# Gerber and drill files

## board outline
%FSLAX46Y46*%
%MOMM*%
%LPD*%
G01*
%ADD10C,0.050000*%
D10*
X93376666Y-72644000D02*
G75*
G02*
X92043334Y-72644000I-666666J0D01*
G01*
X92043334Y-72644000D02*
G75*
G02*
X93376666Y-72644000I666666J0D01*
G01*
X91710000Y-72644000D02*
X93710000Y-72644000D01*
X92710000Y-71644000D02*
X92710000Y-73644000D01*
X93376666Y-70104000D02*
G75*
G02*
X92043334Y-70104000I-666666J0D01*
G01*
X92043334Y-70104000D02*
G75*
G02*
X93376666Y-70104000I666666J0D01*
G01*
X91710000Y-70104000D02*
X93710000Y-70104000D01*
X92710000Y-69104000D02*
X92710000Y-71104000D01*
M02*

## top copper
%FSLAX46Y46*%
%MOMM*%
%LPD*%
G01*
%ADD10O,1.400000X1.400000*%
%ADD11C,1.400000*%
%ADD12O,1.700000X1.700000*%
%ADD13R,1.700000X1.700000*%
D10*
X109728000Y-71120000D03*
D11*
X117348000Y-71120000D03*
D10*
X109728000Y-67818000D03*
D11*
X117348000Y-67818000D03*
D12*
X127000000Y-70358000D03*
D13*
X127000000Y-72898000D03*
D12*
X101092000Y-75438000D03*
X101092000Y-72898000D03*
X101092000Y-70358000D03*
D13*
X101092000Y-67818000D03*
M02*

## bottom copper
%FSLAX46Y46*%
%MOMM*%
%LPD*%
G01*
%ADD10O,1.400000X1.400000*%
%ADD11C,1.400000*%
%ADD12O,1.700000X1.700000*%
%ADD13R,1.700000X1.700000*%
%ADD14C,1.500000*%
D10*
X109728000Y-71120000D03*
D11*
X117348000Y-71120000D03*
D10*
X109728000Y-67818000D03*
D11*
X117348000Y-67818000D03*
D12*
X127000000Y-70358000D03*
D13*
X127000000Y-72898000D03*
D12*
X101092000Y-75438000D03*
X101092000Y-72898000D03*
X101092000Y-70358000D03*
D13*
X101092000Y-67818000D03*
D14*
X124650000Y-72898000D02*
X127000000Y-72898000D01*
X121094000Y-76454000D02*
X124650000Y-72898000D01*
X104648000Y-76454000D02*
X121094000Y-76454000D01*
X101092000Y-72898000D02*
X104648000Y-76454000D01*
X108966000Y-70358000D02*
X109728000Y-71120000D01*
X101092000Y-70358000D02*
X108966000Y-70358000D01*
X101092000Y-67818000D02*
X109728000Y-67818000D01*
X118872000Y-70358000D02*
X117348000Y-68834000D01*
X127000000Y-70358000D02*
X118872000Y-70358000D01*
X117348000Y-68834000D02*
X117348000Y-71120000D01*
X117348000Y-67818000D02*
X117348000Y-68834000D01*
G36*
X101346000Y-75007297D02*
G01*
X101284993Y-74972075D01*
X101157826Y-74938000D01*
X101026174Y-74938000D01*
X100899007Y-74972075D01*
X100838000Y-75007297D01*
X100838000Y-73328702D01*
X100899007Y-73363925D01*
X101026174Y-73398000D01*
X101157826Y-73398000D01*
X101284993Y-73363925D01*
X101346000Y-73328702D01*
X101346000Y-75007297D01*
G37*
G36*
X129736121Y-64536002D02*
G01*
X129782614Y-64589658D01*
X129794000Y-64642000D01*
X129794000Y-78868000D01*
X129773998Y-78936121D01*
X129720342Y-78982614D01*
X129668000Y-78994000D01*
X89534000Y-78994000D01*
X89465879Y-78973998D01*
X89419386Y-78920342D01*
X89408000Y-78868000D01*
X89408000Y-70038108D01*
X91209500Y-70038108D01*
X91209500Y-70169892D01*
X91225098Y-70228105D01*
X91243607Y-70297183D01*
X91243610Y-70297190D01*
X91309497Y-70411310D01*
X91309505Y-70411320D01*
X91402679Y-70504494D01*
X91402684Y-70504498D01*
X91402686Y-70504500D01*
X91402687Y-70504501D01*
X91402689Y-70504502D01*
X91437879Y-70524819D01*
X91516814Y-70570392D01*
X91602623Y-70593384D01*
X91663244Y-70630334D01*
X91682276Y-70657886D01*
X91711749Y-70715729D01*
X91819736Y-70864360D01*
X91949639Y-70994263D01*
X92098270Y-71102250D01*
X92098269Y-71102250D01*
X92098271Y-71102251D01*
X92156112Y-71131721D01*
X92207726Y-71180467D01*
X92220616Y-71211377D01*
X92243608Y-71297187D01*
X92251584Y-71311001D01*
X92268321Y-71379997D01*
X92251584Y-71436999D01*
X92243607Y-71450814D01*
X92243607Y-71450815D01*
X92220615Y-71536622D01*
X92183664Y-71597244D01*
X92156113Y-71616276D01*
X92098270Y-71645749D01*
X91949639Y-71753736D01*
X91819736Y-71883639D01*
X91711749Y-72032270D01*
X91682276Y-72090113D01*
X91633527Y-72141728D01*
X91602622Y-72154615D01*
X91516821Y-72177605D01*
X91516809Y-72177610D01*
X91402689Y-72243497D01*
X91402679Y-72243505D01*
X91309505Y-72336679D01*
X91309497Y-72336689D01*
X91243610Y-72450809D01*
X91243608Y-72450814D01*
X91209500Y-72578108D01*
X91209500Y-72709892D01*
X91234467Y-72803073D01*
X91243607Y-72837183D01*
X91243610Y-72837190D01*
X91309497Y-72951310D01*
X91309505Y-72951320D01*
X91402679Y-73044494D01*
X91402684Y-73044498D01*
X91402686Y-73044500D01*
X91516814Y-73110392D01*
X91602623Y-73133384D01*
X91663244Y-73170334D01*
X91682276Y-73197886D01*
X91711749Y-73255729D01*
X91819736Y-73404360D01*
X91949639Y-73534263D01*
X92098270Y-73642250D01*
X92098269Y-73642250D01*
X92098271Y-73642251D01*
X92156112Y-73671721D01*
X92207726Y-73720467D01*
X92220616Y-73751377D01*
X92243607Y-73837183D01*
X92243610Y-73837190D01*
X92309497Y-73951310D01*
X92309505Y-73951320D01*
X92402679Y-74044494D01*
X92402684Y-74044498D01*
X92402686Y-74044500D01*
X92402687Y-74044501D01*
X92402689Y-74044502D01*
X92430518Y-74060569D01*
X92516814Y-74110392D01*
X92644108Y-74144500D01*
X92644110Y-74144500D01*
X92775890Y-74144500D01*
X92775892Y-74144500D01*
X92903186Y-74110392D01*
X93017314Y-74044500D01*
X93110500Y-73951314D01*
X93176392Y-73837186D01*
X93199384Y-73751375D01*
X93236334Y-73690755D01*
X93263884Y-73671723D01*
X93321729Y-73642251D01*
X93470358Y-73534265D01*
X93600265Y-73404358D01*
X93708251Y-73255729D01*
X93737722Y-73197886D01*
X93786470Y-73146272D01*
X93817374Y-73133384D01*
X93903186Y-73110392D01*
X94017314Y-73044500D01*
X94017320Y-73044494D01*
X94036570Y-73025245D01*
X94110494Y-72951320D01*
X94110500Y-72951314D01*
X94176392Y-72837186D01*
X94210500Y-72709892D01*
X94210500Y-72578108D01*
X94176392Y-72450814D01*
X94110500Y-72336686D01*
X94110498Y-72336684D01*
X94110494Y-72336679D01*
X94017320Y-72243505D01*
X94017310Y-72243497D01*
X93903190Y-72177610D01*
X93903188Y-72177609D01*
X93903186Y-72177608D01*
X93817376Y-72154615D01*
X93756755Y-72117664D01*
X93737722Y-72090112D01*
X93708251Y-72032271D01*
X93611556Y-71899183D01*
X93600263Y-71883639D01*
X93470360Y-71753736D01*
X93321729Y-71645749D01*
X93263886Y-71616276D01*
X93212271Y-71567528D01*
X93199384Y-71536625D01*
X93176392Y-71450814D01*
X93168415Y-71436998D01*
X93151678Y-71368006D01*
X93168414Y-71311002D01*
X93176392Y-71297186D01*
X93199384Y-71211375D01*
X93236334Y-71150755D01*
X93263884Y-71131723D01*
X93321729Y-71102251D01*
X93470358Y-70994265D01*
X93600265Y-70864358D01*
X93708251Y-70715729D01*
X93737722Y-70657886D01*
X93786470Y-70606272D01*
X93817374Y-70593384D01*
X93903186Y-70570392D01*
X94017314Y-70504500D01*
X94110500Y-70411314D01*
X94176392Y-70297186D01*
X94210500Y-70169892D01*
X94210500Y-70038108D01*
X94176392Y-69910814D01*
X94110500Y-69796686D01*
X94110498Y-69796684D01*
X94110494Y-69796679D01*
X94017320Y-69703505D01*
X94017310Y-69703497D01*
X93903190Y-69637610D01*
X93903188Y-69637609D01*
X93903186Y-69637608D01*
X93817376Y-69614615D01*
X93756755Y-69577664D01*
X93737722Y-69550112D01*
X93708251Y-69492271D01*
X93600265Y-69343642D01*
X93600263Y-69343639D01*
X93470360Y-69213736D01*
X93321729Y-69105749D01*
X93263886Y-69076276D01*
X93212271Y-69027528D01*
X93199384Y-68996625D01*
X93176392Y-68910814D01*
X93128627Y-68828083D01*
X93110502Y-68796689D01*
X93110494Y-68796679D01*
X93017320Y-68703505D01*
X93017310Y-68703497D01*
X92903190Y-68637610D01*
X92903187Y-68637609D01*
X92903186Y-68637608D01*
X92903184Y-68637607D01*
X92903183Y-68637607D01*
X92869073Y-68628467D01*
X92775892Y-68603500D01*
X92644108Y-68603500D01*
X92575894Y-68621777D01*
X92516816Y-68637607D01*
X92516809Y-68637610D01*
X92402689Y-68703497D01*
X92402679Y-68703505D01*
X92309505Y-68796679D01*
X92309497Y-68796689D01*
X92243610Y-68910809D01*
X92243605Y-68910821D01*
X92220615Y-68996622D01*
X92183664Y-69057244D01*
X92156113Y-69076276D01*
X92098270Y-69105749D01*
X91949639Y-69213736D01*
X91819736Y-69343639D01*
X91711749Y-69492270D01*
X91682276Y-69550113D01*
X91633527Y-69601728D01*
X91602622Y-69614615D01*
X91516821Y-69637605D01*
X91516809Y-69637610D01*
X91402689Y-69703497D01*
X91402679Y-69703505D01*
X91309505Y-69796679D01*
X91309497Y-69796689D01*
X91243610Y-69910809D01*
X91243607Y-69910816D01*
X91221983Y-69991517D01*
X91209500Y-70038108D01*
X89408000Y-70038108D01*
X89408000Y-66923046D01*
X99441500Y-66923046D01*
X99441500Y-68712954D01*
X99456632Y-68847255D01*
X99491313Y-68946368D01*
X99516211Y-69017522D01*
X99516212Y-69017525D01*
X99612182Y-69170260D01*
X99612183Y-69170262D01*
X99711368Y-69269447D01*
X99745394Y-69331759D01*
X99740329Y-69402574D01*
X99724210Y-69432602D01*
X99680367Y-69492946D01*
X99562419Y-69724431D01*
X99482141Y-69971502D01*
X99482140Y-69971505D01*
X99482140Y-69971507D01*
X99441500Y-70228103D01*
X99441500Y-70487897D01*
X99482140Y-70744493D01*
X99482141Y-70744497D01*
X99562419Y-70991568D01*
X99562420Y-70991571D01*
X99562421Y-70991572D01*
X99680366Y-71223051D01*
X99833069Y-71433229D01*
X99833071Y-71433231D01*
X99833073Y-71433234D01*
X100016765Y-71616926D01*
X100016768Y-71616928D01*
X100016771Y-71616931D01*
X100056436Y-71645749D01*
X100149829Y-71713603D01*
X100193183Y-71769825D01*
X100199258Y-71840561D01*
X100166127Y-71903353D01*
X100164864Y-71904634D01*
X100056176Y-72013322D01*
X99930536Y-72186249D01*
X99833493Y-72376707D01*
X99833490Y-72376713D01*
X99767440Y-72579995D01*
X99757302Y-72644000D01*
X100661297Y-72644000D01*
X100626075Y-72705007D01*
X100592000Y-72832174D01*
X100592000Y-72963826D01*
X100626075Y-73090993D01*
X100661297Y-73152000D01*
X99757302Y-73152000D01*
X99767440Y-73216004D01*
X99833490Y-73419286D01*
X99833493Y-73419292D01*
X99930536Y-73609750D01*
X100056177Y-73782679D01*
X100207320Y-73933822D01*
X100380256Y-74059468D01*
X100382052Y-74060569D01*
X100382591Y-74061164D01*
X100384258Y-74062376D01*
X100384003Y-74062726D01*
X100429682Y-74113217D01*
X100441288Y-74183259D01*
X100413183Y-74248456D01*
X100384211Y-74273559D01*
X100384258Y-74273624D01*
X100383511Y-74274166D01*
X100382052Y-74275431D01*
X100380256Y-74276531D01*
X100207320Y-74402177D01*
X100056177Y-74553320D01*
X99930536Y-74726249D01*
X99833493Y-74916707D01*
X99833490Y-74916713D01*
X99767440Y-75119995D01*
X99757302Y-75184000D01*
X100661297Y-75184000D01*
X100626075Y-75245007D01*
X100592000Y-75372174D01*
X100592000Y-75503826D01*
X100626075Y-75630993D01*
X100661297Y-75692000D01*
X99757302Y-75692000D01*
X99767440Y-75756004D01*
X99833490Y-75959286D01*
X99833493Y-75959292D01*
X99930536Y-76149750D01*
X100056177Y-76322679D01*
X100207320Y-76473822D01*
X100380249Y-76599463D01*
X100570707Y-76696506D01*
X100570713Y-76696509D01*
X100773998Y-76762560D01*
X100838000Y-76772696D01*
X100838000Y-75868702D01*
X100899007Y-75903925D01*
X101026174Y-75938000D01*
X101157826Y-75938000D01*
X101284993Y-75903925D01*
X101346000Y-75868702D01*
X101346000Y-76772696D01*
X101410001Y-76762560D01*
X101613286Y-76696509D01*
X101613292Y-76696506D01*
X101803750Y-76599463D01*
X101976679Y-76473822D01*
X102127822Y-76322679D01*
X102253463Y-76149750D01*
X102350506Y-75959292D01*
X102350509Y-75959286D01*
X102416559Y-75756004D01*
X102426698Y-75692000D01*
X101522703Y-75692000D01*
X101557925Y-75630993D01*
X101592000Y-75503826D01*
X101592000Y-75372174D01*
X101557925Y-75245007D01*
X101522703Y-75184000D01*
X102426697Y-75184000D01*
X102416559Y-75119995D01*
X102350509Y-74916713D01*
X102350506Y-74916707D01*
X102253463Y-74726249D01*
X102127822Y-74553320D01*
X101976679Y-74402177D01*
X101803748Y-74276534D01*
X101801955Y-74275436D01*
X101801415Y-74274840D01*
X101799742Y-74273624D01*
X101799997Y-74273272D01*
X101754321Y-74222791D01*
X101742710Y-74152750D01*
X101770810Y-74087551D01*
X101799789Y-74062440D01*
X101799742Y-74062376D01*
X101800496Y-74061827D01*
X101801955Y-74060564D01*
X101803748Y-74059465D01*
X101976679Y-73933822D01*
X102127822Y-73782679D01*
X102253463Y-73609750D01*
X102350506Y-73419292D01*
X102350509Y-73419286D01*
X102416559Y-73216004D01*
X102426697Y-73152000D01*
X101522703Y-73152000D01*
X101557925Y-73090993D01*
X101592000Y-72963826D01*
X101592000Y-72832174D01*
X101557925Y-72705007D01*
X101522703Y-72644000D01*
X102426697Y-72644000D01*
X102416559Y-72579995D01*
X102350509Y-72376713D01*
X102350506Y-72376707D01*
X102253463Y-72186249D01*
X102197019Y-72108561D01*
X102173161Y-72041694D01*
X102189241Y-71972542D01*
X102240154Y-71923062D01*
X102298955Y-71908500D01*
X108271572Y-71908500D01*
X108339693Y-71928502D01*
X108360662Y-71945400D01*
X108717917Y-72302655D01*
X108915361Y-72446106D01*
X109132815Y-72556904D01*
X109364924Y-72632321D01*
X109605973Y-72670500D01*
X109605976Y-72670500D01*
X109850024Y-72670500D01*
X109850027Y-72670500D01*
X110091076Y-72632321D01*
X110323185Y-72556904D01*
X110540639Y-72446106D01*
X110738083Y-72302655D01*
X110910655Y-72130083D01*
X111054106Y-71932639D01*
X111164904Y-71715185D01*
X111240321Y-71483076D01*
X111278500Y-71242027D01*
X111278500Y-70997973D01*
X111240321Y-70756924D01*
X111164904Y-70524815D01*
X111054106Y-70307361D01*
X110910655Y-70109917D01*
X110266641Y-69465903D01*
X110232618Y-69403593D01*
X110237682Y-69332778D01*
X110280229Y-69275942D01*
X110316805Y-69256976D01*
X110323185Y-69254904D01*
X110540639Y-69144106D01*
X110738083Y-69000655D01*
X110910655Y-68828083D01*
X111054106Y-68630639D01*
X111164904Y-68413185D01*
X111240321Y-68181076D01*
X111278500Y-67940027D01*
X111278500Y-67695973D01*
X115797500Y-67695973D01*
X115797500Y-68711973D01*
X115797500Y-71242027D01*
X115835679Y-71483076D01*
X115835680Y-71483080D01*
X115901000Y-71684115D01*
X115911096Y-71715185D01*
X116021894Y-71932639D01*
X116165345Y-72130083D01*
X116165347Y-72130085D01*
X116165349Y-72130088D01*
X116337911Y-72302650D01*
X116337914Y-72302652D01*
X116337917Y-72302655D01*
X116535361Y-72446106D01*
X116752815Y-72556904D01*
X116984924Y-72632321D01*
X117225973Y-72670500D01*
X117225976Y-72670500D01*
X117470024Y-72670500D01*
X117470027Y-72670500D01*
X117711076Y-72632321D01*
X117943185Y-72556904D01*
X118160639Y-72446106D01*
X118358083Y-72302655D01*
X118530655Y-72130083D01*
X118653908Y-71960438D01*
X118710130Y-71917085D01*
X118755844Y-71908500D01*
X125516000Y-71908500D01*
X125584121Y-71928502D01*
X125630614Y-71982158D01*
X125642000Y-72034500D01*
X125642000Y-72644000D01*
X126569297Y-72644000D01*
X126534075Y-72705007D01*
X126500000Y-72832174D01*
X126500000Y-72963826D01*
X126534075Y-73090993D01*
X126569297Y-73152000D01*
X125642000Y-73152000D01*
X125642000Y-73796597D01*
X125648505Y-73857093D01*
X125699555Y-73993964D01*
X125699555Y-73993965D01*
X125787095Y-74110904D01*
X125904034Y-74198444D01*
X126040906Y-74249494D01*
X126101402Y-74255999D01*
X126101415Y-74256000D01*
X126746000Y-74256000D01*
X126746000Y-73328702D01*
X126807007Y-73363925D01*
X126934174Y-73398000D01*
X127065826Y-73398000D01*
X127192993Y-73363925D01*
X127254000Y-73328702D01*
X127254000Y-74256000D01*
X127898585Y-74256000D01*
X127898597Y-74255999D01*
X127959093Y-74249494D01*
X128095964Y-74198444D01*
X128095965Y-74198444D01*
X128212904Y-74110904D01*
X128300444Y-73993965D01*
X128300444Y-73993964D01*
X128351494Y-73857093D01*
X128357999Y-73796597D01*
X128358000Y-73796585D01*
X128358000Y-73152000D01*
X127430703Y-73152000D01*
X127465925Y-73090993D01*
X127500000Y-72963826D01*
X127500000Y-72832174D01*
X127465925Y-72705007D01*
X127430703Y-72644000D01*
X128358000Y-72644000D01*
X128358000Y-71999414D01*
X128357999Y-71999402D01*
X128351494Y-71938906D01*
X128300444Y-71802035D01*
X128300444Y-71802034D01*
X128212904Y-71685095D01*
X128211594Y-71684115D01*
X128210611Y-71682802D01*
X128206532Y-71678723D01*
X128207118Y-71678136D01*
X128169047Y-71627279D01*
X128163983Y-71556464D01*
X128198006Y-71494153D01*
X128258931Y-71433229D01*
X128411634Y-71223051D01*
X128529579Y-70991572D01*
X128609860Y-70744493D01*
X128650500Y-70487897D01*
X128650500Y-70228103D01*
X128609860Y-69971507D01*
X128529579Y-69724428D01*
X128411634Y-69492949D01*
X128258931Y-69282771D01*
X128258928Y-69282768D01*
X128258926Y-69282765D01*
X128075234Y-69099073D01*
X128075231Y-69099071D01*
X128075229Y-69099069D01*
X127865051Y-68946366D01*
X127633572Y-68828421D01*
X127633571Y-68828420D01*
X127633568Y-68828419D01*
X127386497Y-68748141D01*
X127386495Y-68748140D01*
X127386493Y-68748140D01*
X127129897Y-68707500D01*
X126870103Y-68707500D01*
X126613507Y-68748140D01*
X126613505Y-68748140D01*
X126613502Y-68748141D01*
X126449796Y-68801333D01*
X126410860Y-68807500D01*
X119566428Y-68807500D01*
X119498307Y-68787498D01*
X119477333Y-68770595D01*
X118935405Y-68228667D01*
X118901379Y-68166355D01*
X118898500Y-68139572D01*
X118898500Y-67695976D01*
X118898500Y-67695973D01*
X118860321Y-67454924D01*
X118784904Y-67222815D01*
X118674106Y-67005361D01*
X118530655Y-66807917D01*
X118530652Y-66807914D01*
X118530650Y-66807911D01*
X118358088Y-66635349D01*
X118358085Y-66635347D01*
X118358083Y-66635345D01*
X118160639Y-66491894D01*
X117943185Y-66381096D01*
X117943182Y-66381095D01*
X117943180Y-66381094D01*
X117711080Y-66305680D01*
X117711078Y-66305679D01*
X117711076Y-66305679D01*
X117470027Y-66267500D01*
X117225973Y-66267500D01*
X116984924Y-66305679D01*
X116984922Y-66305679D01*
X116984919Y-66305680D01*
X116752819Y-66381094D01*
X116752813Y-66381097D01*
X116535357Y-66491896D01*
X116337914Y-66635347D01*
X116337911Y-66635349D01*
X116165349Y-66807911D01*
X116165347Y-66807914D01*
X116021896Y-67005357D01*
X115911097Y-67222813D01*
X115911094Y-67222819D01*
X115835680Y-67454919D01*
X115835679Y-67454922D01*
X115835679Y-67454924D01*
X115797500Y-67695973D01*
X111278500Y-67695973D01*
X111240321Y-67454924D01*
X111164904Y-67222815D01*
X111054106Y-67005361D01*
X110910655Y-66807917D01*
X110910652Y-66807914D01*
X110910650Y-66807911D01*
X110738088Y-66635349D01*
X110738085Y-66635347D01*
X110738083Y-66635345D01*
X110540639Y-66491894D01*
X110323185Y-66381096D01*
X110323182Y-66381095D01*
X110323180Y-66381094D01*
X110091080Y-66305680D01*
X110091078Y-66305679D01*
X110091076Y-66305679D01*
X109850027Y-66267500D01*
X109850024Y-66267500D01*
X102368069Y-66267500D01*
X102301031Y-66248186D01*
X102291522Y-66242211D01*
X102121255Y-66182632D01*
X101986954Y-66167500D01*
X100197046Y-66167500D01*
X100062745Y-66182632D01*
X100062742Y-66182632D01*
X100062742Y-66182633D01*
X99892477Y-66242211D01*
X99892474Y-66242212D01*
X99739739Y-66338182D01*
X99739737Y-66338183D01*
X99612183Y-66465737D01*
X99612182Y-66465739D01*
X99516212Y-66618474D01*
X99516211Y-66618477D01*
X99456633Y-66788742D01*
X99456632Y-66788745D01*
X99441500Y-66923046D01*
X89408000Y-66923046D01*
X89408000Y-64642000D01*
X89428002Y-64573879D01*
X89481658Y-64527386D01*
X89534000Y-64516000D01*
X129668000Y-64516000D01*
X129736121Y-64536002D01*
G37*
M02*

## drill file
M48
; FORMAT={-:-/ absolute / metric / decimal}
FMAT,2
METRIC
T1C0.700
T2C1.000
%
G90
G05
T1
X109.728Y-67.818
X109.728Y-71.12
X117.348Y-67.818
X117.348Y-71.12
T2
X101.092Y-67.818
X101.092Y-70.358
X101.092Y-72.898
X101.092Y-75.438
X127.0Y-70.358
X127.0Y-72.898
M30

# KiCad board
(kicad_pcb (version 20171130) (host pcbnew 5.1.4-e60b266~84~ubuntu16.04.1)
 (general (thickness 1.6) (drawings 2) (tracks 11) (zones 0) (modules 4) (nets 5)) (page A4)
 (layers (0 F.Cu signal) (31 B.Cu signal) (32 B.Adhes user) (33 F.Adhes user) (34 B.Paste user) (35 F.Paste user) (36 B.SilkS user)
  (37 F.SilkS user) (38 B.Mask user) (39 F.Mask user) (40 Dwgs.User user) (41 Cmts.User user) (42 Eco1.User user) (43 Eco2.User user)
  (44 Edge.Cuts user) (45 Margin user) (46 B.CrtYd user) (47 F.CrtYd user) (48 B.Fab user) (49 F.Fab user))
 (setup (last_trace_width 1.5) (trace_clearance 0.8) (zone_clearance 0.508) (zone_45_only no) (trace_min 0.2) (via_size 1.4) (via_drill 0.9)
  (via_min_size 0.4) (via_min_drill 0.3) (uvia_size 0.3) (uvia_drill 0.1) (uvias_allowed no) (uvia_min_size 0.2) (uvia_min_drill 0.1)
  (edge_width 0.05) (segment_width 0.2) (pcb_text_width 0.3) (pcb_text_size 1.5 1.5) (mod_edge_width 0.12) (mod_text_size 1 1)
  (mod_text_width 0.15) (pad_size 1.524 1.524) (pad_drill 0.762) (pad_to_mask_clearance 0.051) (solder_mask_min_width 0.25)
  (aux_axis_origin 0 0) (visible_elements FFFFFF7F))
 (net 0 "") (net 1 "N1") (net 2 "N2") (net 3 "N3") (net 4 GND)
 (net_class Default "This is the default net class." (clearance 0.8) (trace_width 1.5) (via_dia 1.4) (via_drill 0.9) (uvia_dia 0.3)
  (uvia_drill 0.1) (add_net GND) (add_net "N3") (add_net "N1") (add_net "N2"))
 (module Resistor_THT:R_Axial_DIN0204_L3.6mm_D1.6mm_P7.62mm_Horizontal (layer F.Cu) (at 117.348 71.12 180)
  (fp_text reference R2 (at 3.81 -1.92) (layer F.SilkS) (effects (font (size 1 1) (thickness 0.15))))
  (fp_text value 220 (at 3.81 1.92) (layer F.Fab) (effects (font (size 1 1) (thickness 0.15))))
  (pad 2 thru_hole oval (at 7.62 0 180) (size 1.4 1.4) (drill 0.7) (layers *.Cu *.Mask) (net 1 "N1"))
  (pad 1 thru_hole circle (at 0 0 180) (size 1.4 1.4) (drill 0.7) (layers *.Cu *.Mask) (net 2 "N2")))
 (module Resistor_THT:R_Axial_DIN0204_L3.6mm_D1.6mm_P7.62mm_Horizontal (layer F.Cu) (at 117.348 67.818 180)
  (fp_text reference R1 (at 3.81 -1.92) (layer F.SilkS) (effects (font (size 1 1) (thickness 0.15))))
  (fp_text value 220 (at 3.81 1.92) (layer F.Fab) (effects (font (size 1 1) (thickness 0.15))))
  (pad 2 thru_hole oval (at 7.62 0 180) (size 1.4 1.4) (drill 0.7) (layers *.Cu *.Mask) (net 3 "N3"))
  (pad 1 thru_hole circle (at 0 0 180) (size 1.4 1.4) (drill 0.7) (layers *.Cu *.Mask) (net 2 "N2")))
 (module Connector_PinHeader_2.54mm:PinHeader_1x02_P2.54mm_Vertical (layer F.Cu) (at 127 72.898 180)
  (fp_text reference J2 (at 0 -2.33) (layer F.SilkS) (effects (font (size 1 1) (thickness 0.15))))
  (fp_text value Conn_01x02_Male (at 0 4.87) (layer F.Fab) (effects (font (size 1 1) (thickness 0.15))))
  (pad 2 thru_hole oval (at 0 2.54 180) (size 1.7 1.7) (drill 1) (layers *.Cu *.Mask) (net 2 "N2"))
  (pad 1 thru_hole rect (at 0 0 180) (size 1.7 1.7) (drill 1) (layers *.Cu *.Mask) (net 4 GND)))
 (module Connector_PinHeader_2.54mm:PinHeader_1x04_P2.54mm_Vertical (layer F.Cu) (at 101.092 67.818)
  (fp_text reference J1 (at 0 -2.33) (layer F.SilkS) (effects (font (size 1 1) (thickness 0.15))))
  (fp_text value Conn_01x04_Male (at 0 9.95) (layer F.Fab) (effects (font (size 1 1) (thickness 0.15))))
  (pad 4 thru_hole oval (at 0 7.62) (size 1.7 1.7) (drill 1) (layers *.Cu *.Mask) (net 4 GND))
  (pad 3 thru_hole oval (at 0 5.08) (size 1.7 1.7) (drill 1) (layers *.Cu *.Mask) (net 4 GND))
  (pad 2 thru_hole oval (at 0 2.54) (size 1.7 1.7) (drill 1) (layers *.Cu *.Mask) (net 1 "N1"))
  (pad 1 thru_hole rect (at 0 0) (size 1.7 1.7) (drill 1) (layers *.Cu *.Mask) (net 3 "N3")))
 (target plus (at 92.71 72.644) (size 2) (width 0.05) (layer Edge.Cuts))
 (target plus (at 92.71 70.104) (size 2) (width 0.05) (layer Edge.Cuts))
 (segment (start 124.65 72.898) (end 127 72.898) (width 1.5) (layer B.Cu) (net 4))
 (segment (start 121.094 76.454) (end 124.65 72.898) (width 1.5) (layer B.Cu) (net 4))
 (segment (start 104.648 76.454) (end 121.094 76.454) (width 1.5) (layer B.Cu) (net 4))
 (segment (start 101.092 72.898) (end 104.648 76.454) (width 1.5) (layer B.Cu) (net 4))
 (segment (start 108.966 70.358) (end 109.728 71.12) (width 1.5) (layer B.Cu) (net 1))
 (segment (start 101.092 70.358) (end 108.966 70.358) (width 1.5) (layer B.Cu) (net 1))
 (segment (start 101.092 67.818) (end 109.728 67.818) (width 1.5) (layer B.Cu) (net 3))
 (segment (start 118.872 70.358) (end 117.348 68.834) (width 1.5) (layer B.Cu) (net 2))
 (segment (start 127 70.358) (end 118.872 70.358) (width 1.5) (layer B.Cu) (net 2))
 (segment (start 117.348 68.834) (end 117.348 71.12) (width 1.5) (layer B.Cu) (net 2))
 (segment (start 117.348 67.818) (end 117.348 68.834) (width 1.5) (layer B.Cu) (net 2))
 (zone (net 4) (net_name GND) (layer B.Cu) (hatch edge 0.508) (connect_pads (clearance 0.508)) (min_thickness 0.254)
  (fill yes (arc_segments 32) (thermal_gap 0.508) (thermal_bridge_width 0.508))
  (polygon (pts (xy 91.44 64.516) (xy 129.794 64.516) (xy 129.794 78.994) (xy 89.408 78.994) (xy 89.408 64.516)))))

